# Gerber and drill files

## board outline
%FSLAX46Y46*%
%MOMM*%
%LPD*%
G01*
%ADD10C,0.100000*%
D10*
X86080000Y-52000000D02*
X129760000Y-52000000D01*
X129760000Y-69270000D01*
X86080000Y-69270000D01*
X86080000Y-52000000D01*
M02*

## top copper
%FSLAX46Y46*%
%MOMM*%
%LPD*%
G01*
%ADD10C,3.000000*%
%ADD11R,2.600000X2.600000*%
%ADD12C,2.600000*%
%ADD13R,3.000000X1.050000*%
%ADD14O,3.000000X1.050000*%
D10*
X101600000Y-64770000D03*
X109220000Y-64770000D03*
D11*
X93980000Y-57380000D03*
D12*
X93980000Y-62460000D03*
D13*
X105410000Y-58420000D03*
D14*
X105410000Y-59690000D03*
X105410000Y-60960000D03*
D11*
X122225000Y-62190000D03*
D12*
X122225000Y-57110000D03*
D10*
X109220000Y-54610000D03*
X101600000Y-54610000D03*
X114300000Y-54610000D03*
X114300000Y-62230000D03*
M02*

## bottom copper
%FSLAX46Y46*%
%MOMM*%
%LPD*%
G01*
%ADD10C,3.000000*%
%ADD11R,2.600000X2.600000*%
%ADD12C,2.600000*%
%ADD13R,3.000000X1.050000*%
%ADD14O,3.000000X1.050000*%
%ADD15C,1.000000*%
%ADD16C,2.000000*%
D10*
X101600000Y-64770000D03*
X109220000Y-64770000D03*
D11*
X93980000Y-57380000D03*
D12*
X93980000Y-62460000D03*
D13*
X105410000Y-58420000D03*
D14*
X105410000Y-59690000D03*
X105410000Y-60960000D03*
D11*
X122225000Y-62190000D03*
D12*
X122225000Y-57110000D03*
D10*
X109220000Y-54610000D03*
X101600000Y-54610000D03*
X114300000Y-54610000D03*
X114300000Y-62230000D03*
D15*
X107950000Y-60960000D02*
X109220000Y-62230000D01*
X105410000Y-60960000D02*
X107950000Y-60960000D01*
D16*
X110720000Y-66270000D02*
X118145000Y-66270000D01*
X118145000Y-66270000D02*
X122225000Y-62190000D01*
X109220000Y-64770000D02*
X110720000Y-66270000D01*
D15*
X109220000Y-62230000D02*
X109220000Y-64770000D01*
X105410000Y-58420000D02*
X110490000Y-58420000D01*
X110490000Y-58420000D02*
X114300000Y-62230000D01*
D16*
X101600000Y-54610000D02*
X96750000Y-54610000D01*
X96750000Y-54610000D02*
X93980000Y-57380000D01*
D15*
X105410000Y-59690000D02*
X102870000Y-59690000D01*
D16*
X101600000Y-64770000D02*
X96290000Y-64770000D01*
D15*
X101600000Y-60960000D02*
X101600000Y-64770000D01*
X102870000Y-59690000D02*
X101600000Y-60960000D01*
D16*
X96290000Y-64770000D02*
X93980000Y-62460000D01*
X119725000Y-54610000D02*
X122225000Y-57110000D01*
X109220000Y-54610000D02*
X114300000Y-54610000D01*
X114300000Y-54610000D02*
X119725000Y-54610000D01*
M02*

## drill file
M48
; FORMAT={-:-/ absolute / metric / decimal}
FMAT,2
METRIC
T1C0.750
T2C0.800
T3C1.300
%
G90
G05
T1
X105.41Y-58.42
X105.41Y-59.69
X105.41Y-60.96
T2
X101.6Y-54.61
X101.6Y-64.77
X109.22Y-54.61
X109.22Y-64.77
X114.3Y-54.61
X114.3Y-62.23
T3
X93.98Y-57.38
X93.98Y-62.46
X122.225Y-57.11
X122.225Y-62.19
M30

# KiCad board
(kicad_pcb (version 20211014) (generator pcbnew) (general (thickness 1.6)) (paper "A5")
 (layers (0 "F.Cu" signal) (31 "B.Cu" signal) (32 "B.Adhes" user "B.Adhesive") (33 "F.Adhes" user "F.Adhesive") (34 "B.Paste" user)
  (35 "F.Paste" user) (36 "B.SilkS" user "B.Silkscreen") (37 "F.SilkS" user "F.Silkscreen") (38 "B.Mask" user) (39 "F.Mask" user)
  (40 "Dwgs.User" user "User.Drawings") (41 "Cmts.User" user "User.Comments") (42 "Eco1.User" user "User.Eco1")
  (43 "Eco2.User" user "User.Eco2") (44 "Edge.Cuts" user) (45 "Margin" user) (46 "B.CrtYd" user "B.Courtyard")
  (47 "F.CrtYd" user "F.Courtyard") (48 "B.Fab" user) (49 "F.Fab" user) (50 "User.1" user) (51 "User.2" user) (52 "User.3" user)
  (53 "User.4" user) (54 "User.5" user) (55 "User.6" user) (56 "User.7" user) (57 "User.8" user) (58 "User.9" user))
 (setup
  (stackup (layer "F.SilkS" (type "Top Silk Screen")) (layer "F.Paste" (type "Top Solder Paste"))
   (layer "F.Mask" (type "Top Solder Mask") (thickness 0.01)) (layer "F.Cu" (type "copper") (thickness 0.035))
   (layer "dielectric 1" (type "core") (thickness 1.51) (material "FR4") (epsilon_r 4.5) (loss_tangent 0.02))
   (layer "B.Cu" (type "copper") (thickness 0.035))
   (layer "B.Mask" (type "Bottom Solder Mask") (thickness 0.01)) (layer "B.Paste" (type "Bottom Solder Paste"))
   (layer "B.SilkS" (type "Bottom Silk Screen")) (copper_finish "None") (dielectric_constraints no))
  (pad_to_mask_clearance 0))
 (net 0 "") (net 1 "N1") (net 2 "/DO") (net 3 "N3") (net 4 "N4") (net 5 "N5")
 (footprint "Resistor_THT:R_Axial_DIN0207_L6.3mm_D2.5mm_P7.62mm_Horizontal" (layer "F.Cu") (at 101.6 64.77)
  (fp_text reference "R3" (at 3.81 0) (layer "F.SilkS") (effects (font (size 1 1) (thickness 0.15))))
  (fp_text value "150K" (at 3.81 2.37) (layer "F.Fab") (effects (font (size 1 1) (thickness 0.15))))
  (pad "1" thru_hole circle (at 0 0) (size 3 3) (drill 0.8) (layers *.Cu *.Mask) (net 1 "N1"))
  (pad "2" thru_hole circle (at 7.62 0) (size 3 3) (drill 0.8) (layers *.Cu *.Mask) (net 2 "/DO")))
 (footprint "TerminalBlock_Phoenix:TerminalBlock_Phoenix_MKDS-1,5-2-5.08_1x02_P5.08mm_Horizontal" (layer "F.Cu") (at 93.98 57.38 -90)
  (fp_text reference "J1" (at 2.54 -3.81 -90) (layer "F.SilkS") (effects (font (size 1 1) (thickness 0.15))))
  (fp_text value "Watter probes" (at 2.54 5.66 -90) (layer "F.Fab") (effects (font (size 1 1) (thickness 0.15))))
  (pad "1" thru_hole rect (at 0 0 270) (size 2.6 2.6) (drill 1.3) (layers *.Cu *.Mask) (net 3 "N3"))
  (pad "2" thru_hole circle (at 5.08 0 270) (size 2.6 2.6) (drill 1.3) (layers *.Cu *.Mask) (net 1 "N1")))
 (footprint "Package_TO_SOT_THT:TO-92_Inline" (layer "F.Cu") (at 105.41 58.42 -90)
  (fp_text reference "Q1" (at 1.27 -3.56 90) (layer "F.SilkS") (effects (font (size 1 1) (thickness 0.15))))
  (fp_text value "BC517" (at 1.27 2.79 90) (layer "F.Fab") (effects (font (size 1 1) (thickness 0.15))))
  (pad "1" thru_hole rect (at 0 0 270) (size 1.05 3) (drill 0.75) (layers *.Cu *.Mask) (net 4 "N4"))
  (pad "2" thru_hole oval (at 1.27 0 270) (size 1.05 3) (drill 0.75) (layers *.Cu *.Mask) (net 1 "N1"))
  (pad "3" thru_hole oval (at 2.54 0 270) (size 1.05 3) (drill 0.75) (layers *.Cu *.Mask) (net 2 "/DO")))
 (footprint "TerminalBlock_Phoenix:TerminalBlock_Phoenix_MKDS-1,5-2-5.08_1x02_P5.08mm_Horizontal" (layer "F.Cu") (at 122.225 62.19 90)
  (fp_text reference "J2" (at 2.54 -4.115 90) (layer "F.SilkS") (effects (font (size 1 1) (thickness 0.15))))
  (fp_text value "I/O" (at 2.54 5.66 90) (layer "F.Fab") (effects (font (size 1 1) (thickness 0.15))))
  (pad "1" thru_hole rect (at 0 0 90) (size 2.6 2.6) (drill 1.3) (layers *.Cu *.Mask) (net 2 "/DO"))
  (pad "2" thru_hole circle (at 5.08 0 90) (size 2.6 2.6) (drill 1.3) (layers *.Cu *.Mask) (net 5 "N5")))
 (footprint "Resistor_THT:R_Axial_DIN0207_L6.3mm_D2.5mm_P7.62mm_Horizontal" (layer "F.Cu") (at 109.22 54.61 180)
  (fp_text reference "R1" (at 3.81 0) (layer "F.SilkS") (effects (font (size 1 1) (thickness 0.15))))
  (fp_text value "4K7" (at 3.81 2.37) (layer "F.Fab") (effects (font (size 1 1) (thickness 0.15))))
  (pad "1" thru_hole circle (at 0 0 180) (size 3 3) (drill 0.8) (layers *.Cu *.Mask) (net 5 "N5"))
  (pad "2" thru_hole circle (at 7.62 0 180) (size 3 3) (drill 0.8) (layers *.Cu *.Mask) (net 3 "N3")))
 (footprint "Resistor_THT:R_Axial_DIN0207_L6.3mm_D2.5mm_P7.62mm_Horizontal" (layer "F.Cu") (at 114.3 54.61 -90)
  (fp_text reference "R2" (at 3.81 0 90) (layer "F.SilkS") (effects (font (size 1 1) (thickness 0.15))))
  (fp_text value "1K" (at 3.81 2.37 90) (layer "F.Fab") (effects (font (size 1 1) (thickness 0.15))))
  (pad "1" thru_hole circle (at 0 0 270) (size 3 3) (drill 0.8) (layers *.Cu *.Mask) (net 5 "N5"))
  (pad "2" thru_hole circle (at 7.62 0 270) (size 3 3) (drill 0.8) (layers *.Cu *.Mask) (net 4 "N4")))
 (gr_rect (start 86.08 52) (end 129.76 69.27) (layer "Edge.Cuts") (width 0.1) (fill none))
 (segment (start 107.95 60.96) (end 109.22 62.23) (width 1) (layer "B.Cu") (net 2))
 (segment (start 105.41 60.96) (end 107.95 60.96) (width 1) (layer "B.Cu") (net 2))
 (segment (start 110.72 66.27) (end 118.145 66.27) (width 2) (layer "B.Cu") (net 2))
 (segment (start 118.145 66.27) (end 122.225 62.19) (width 2) (layer "B.Cu") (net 2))
 (segment (start 109.22 64.77) (end 110.72 66.27) (width 2) (layer "B.Cu") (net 2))
 (segment (start 109.22 62.23) (end 109.22 64.77) (width 1) (layer "B.Cu") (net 2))
 (segment (start 105.41 58.42) (end 110.49 58.42) (width 1) (layer "B.Cu") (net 4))
 (segment (start 110.49 58.42) (end 114.3 62.23) (width 1) (layer "B.Cu") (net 4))
 (segment (start 101.6 54.61) (end 96.75 54.61) (width 2) (layer "B.Cu") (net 3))
 (segment (start 96.75 54.61) (end 93.98 57.38) (width 2) (layer "B.Cu") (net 3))
 (segment (start 105.41 59.69) (end 102.87 59.69) (width 1) (layer "B.Cu") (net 1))
 (segment (start 101.6 64.77) (end 96.29 64.77) (width 2) (layer "B.Cu") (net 1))
 (segment (start 101.6 60.96) (end 101.6 64.77) (width 1) (layer "B.Cu") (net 1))
 (segment (start 102.87 59.69) (end 101.6 60.96) (width 1) (layer "B.Cu") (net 1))
 (segment (start 96.29 64.77) (end 93.98 62.46) (width 2) (layer "B.Cu") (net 1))
 (segment (start 119.725 54.61) (end 122.225 57.11) (width 2) (layer "B.Cu") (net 5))
 (segment (start 109.22 54.61) (end 114.3 54.61) (width 2) (layer "B.Cu") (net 5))
 (segment (start 114.3 54.61) (end 119.725 54.61) (width 2) (layer "B.Cu") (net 5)))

